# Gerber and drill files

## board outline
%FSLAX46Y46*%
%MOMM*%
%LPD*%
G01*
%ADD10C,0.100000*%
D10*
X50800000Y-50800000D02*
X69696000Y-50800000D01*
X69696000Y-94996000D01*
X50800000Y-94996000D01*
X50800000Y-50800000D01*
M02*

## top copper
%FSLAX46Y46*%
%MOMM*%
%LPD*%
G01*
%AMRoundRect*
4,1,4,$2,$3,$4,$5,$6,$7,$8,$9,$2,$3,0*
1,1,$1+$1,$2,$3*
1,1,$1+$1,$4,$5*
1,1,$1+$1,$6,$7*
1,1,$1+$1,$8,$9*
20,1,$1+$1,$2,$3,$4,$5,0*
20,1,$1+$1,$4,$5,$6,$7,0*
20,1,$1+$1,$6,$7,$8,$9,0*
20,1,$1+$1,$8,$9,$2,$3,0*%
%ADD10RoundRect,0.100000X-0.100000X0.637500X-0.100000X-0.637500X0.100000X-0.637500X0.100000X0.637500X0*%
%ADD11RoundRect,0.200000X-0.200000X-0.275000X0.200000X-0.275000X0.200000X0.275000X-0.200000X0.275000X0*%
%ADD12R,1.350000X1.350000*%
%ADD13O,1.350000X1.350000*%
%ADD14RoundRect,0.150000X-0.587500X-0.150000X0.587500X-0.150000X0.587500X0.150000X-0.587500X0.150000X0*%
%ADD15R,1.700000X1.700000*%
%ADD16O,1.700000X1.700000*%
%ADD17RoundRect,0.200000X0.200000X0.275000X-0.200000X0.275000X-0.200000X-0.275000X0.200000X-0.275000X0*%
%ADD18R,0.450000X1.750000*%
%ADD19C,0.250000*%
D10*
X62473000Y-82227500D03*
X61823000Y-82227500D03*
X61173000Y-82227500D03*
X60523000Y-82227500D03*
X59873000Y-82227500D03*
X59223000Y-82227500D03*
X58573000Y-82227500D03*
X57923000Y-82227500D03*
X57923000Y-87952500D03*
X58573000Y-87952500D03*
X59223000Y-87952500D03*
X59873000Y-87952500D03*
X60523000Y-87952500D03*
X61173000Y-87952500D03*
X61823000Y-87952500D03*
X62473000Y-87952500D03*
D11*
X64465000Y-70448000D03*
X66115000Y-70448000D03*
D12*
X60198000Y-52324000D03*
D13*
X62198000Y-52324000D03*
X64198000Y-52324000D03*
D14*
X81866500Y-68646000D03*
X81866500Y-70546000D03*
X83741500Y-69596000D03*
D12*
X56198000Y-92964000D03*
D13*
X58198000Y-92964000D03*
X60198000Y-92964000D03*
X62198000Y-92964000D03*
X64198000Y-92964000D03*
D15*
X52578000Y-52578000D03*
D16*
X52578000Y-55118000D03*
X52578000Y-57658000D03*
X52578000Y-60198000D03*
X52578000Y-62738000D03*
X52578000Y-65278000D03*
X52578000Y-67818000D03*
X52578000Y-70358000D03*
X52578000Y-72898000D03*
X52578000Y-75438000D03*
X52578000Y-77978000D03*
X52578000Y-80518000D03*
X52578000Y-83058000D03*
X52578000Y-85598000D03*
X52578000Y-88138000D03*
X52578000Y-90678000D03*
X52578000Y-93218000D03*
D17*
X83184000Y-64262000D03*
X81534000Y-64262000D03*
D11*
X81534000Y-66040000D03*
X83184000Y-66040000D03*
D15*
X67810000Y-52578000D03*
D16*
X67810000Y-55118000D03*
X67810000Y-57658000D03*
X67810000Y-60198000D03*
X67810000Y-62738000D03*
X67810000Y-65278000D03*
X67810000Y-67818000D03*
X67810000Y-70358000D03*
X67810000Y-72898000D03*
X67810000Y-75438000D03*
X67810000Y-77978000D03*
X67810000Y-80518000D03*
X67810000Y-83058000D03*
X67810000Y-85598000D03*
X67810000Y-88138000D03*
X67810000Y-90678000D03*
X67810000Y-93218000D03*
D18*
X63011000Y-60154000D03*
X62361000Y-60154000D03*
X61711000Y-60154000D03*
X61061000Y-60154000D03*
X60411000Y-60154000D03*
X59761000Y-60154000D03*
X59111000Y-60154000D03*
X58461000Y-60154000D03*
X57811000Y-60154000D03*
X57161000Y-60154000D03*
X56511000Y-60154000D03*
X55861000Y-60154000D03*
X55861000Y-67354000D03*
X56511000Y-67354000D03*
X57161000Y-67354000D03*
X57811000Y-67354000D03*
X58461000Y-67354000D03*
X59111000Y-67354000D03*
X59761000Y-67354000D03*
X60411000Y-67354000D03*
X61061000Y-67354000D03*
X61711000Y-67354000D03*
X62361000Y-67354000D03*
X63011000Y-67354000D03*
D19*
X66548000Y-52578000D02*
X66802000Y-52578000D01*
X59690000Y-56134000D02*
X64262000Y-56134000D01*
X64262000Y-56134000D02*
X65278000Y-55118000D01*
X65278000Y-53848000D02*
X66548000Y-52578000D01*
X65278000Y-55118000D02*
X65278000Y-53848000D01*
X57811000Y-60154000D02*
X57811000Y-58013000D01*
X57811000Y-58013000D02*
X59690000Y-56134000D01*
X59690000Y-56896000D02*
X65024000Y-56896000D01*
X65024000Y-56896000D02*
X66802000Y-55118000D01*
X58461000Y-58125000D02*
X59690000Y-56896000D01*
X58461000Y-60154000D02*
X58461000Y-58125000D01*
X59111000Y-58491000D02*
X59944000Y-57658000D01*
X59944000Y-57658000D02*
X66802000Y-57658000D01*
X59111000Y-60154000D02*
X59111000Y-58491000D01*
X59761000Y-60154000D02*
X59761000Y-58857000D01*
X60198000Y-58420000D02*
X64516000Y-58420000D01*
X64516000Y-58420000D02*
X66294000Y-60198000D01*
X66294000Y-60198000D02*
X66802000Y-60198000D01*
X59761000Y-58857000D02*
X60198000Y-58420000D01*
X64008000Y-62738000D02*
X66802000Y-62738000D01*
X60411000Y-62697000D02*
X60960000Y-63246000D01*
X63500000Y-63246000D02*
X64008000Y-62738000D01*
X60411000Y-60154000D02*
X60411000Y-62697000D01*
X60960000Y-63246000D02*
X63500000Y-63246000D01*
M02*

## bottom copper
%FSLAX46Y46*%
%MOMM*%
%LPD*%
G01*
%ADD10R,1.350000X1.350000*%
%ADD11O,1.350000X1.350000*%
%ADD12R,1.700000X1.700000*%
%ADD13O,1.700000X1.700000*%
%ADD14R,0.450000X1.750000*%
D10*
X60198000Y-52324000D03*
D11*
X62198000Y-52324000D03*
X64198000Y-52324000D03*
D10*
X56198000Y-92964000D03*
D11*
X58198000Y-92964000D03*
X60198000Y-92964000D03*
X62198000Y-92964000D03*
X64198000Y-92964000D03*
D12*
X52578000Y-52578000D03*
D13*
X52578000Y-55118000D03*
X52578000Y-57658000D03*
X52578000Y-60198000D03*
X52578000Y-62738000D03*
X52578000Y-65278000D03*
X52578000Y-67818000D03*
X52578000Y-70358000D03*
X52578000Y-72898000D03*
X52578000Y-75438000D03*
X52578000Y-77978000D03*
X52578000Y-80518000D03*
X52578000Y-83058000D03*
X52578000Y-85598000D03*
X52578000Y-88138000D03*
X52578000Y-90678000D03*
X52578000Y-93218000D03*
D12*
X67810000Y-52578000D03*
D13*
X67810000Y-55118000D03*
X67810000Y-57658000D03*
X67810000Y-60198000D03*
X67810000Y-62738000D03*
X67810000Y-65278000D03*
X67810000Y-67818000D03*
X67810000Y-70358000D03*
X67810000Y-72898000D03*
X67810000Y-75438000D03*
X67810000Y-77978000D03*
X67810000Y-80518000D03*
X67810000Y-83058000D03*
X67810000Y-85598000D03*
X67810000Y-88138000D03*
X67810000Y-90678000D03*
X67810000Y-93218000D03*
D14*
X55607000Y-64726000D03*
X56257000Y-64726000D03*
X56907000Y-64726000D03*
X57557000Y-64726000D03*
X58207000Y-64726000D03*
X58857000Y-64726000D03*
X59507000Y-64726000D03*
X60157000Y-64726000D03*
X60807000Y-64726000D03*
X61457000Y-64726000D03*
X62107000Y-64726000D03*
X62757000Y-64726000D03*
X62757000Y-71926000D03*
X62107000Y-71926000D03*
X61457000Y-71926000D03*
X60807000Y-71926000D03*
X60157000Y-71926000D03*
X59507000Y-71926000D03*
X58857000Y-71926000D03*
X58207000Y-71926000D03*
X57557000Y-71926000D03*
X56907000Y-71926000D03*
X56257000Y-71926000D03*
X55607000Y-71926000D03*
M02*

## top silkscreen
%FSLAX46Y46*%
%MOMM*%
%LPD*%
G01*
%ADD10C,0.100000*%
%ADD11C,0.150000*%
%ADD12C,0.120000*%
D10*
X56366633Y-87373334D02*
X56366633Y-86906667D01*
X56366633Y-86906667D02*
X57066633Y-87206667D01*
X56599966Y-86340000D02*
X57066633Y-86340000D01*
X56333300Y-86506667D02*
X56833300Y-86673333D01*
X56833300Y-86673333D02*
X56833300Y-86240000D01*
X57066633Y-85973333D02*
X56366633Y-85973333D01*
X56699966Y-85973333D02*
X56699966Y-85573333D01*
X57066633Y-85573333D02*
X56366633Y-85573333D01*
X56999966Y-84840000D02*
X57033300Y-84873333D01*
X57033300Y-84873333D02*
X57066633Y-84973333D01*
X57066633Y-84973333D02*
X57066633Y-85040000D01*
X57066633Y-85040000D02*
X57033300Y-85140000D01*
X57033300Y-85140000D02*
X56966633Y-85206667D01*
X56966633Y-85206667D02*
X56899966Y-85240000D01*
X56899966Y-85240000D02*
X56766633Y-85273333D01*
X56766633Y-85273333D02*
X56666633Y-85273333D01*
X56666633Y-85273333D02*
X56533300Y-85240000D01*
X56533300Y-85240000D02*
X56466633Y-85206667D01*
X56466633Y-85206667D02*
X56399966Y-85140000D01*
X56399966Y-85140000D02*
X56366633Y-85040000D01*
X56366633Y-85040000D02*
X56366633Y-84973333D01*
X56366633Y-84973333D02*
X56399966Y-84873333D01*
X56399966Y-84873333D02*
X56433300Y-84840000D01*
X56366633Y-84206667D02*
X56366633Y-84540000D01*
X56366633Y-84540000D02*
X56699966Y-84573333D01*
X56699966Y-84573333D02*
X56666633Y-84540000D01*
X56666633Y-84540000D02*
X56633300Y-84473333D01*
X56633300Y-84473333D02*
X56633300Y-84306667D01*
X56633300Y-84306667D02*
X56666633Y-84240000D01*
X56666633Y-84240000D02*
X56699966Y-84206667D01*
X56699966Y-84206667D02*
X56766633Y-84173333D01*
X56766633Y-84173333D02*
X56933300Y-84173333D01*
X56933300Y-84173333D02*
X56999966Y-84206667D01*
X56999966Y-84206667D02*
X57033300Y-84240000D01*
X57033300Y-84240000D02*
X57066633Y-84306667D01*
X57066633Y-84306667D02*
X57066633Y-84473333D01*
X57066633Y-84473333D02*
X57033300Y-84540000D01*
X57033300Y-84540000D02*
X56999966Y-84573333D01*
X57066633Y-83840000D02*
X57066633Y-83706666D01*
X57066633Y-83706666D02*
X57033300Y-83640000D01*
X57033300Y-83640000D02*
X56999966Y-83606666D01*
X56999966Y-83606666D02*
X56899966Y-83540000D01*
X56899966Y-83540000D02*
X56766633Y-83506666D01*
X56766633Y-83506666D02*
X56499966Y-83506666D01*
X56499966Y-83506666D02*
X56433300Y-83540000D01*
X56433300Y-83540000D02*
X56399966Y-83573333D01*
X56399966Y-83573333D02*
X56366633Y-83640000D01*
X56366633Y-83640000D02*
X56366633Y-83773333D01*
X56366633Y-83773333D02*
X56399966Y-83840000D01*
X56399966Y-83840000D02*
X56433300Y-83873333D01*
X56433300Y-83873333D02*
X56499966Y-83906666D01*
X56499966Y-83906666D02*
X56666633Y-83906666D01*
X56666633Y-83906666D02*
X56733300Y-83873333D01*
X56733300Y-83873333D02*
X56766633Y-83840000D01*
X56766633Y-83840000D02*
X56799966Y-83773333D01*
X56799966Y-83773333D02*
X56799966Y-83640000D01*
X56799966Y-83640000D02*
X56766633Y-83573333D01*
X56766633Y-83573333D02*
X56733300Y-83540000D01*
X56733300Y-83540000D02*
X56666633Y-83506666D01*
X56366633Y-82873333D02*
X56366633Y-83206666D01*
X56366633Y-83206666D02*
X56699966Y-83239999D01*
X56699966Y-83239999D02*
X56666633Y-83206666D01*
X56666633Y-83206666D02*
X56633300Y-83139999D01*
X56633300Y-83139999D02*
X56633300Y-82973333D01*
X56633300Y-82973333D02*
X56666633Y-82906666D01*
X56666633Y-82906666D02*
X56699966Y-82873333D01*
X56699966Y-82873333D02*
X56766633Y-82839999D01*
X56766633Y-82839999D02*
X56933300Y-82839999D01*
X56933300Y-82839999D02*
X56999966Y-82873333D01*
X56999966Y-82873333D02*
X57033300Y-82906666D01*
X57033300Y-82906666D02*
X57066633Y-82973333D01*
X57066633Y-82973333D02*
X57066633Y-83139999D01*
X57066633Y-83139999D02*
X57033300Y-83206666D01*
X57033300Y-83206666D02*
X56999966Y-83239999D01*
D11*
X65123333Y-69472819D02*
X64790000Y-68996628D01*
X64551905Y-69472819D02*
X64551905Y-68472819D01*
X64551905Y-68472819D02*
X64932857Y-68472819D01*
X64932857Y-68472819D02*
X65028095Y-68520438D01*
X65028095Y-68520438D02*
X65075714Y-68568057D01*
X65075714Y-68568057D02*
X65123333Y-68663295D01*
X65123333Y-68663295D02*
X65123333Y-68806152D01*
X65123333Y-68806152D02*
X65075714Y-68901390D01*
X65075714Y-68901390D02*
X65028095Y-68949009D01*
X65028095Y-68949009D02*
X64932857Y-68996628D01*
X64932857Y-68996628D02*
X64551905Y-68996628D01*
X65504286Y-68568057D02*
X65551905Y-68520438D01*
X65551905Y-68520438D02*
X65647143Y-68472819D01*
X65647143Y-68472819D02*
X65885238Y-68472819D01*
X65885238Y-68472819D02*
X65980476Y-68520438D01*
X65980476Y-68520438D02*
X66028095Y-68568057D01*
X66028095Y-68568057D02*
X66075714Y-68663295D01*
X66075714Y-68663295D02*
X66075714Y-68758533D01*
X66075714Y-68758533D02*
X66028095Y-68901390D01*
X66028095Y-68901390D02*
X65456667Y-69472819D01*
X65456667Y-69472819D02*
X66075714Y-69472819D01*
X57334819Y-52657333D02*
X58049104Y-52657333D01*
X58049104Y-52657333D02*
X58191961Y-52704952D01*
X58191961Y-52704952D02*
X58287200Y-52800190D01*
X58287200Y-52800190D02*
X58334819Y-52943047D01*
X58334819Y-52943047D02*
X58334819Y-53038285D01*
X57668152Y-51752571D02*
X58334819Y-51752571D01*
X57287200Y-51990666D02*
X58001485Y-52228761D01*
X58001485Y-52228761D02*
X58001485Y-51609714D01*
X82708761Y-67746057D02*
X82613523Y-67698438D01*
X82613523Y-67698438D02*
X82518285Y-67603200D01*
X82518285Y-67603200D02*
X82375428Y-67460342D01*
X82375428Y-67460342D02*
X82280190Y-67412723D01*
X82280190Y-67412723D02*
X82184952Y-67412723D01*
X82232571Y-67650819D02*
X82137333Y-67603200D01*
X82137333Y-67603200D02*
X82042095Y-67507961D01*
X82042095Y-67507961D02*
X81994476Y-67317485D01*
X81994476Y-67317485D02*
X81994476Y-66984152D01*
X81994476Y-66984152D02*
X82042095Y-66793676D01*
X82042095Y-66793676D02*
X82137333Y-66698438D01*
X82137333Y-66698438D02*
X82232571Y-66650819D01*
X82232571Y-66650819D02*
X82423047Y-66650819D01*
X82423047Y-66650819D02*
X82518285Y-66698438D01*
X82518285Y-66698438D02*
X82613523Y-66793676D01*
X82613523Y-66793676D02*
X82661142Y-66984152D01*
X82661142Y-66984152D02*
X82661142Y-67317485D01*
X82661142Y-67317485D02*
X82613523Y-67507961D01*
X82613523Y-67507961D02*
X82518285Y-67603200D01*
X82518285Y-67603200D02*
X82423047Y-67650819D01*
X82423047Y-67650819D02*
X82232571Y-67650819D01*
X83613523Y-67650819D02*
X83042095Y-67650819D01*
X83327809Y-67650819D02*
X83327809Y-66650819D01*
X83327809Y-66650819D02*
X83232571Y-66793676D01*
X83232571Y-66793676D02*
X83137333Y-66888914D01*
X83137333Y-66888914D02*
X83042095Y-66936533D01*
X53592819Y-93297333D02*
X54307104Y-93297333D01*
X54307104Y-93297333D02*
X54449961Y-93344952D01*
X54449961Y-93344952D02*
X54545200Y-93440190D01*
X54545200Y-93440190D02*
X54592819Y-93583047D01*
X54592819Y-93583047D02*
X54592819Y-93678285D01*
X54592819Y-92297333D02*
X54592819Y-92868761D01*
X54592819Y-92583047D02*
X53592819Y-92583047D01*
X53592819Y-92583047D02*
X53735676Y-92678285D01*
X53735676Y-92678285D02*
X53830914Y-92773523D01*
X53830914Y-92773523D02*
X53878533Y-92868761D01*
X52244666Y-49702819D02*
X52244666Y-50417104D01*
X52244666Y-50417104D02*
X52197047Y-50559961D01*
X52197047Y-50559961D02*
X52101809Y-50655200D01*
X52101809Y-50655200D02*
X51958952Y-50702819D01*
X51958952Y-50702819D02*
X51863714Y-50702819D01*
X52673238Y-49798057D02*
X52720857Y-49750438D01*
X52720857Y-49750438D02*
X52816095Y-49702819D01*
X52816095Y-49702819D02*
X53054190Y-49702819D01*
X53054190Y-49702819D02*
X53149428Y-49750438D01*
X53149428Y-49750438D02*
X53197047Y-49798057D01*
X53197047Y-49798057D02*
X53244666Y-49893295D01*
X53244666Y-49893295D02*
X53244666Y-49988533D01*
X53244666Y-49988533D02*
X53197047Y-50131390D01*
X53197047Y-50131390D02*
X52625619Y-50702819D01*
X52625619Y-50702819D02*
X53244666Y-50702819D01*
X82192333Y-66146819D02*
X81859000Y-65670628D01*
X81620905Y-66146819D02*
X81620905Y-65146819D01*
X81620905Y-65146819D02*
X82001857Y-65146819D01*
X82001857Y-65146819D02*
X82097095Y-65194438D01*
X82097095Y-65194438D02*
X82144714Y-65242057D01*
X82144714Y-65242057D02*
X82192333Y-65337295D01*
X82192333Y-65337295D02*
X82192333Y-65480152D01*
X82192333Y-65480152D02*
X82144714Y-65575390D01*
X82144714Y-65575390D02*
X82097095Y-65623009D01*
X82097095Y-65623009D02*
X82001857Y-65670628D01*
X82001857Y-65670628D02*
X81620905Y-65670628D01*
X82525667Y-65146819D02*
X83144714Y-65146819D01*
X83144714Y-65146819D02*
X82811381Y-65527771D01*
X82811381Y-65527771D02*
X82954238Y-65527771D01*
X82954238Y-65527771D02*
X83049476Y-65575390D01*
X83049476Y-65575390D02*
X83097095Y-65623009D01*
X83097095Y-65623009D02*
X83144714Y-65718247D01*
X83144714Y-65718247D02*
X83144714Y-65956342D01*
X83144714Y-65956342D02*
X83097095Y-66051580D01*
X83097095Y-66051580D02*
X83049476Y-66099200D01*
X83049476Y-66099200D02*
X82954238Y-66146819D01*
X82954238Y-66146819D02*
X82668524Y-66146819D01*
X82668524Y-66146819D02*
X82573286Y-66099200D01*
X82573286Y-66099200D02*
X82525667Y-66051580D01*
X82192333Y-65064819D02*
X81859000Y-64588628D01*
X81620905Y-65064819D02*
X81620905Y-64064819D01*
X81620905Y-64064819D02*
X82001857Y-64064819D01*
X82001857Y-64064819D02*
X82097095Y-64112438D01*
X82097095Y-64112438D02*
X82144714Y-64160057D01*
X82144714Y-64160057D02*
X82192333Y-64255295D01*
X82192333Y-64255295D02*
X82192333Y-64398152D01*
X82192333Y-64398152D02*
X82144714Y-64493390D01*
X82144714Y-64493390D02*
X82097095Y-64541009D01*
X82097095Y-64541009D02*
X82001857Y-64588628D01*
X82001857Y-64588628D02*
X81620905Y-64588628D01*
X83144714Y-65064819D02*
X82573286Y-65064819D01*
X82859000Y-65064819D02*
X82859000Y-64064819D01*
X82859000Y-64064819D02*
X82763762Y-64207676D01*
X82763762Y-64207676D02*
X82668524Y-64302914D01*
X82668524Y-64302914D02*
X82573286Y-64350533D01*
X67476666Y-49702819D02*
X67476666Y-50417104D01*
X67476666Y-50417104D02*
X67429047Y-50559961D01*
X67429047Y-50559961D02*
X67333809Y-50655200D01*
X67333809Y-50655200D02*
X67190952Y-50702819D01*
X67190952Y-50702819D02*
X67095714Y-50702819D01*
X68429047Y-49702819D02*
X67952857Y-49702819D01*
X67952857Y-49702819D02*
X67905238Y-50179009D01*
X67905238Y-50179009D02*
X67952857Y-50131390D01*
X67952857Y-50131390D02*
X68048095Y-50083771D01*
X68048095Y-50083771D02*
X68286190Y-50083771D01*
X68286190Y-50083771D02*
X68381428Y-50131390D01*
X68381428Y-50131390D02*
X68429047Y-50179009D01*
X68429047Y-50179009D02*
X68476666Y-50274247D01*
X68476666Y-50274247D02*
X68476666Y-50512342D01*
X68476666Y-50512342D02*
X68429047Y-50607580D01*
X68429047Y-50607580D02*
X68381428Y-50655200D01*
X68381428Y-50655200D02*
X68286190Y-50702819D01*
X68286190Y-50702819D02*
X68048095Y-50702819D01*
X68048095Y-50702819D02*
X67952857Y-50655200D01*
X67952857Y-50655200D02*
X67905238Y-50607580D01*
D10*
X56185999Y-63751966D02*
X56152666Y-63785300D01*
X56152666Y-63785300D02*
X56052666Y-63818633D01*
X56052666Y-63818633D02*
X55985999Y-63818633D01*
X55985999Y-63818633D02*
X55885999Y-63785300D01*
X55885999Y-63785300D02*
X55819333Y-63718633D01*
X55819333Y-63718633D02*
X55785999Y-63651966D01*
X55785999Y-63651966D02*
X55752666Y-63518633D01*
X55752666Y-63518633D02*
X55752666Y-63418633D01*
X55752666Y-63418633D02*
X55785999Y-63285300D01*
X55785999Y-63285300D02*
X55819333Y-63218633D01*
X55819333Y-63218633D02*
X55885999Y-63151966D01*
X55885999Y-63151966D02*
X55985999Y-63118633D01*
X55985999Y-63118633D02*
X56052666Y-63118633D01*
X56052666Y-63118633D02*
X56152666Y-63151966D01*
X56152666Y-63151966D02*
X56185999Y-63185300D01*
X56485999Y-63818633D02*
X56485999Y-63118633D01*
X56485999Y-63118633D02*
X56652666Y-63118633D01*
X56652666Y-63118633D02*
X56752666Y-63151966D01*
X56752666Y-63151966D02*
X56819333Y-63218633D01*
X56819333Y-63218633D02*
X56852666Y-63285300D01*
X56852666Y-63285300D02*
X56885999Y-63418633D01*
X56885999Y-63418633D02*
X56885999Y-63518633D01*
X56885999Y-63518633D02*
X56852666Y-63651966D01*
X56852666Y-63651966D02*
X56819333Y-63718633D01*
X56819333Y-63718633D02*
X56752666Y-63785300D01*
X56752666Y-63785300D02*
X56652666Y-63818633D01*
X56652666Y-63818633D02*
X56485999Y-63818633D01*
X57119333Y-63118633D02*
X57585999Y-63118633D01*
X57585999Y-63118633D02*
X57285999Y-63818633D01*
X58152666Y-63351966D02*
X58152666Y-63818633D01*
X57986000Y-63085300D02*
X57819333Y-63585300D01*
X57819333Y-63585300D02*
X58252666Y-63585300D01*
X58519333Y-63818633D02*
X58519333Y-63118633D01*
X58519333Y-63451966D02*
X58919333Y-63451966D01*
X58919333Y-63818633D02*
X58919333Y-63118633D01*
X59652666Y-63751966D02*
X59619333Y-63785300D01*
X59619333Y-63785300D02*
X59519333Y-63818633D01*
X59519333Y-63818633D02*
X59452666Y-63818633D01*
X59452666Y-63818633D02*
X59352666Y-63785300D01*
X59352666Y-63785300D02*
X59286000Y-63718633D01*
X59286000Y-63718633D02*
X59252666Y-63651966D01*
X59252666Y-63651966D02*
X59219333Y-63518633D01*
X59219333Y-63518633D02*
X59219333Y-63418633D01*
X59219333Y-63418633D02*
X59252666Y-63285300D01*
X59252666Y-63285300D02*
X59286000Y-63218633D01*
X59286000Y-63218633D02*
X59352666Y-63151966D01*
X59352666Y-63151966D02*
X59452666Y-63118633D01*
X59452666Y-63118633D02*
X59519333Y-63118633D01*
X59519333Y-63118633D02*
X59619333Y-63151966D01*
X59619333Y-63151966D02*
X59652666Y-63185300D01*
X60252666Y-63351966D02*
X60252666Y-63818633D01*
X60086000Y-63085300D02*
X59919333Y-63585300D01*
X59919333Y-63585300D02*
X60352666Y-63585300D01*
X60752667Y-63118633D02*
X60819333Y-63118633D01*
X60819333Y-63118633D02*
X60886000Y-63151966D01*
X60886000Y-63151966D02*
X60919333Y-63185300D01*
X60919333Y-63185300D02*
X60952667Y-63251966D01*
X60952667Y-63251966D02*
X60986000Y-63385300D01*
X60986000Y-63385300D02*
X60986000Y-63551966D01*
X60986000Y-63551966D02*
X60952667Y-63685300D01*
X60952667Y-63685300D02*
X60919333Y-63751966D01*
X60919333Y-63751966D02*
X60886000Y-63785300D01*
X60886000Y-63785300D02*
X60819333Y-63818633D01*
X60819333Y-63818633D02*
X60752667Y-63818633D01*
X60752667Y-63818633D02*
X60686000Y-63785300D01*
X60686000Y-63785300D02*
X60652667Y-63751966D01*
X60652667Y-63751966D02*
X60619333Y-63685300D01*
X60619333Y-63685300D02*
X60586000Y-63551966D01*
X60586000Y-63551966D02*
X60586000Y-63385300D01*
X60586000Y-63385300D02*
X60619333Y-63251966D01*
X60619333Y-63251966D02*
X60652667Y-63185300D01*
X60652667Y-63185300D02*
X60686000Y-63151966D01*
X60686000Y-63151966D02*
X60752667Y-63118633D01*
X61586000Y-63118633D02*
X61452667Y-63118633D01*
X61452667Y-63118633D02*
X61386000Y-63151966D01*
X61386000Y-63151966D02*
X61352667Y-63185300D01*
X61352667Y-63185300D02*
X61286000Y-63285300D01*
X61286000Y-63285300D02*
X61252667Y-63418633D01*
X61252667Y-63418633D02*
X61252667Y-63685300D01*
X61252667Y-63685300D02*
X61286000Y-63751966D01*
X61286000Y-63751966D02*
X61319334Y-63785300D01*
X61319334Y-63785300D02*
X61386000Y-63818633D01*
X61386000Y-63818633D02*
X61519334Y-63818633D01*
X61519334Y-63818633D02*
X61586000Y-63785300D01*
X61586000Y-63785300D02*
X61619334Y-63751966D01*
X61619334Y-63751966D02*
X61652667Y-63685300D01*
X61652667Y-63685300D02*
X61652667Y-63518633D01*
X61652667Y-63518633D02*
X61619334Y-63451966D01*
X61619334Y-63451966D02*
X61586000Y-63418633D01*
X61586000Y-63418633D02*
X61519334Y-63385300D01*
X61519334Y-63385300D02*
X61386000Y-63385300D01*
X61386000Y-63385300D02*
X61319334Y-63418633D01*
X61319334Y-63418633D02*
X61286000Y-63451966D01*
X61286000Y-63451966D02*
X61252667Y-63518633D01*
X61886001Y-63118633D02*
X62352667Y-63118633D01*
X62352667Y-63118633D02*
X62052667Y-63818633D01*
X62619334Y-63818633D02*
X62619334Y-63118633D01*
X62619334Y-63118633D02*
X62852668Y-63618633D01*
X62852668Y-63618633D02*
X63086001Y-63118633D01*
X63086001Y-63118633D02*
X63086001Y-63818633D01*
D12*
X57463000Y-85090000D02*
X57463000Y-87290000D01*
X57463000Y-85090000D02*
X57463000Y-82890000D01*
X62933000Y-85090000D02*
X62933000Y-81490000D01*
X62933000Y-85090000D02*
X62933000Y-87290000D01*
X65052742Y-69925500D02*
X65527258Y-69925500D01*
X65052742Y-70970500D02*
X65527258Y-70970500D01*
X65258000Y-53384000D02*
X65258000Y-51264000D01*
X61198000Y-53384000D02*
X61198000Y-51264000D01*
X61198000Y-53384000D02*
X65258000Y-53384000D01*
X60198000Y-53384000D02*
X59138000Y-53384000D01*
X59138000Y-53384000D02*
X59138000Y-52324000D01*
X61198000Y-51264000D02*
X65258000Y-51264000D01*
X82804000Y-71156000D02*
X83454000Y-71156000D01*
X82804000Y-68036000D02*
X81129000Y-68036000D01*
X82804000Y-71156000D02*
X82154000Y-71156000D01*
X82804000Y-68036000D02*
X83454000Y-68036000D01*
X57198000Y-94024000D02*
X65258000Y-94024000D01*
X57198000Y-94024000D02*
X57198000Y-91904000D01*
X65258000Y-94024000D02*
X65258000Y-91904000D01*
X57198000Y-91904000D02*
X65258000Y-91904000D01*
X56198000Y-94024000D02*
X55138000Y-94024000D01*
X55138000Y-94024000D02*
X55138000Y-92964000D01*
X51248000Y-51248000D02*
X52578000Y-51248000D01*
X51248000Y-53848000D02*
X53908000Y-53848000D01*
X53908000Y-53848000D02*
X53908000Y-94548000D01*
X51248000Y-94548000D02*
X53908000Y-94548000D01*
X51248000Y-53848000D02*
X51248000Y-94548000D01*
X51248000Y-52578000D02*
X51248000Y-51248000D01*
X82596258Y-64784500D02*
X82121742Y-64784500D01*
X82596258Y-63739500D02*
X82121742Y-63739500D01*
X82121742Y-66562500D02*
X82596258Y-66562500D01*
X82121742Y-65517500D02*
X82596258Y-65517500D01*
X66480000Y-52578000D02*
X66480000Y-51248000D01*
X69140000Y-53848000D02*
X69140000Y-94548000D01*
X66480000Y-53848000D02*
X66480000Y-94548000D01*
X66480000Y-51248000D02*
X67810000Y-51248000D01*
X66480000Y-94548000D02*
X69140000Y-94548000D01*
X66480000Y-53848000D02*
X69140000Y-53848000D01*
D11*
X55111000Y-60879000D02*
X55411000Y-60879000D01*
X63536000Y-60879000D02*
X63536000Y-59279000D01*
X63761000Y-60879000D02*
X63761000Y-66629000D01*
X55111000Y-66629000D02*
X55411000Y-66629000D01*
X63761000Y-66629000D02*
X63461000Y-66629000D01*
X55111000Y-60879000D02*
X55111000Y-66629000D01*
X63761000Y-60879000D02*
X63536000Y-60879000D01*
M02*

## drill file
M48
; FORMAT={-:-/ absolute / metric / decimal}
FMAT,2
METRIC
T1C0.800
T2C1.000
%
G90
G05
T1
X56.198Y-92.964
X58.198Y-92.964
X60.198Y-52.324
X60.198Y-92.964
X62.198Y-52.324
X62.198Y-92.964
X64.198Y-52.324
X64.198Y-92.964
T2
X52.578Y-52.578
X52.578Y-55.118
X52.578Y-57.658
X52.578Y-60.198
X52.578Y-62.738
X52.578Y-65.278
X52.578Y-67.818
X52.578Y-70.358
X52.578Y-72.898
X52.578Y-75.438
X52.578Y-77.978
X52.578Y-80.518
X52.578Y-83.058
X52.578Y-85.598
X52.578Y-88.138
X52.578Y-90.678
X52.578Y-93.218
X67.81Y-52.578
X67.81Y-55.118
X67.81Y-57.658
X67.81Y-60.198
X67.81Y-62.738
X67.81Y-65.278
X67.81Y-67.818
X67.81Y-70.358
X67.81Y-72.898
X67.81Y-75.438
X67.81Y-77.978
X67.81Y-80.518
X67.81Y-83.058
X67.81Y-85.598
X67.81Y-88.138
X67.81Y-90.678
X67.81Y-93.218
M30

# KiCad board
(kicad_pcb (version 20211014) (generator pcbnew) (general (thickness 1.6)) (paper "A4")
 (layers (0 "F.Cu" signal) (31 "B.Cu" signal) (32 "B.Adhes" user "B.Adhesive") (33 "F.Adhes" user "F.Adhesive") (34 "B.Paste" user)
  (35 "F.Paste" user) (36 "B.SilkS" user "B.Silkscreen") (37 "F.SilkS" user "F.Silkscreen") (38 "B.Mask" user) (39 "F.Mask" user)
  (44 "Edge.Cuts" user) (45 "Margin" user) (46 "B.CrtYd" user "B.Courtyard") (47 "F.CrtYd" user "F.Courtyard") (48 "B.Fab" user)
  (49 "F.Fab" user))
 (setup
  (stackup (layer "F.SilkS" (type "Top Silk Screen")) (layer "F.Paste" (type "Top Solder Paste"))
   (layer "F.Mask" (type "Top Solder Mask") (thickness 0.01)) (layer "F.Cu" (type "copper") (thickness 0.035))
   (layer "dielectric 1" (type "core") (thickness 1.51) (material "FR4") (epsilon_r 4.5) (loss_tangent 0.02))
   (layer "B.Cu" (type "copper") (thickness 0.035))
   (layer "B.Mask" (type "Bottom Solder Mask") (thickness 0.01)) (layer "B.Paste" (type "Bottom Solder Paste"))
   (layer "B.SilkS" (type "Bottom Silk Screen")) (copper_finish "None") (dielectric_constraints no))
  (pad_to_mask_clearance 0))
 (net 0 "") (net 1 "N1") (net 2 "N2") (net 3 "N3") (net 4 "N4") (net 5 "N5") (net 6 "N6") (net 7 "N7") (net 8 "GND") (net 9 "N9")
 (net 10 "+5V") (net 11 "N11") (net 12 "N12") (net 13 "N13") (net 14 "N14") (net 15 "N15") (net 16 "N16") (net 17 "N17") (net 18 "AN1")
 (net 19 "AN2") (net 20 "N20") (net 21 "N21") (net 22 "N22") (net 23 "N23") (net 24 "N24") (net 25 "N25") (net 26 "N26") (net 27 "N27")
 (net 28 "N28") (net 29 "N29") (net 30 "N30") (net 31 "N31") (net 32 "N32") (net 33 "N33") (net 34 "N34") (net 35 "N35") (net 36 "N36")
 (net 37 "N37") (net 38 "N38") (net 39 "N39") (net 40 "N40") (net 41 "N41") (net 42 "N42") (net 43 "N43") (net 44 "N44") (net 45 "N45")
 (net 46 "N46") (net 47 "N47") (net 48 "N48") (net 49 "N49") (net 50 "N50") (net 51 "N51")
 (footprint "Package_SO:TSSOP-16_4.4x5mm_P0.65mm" (layer "F.Cu") (at 60.198 85.09 -90)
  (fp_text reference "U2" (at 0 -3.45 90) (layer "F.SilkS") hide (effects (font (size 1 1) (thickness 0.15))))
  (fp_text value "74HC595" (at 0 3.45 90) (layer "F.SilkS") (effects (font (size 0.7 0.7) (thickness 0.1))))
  (fp_line (start 0 2.735) (end 2.2 2.735) (layer "F.SilkS") (width 0.12))
  (fp_line (start 0 2.735) (end -2.2 2.735) (layer "F.SilkS") (width 0.12))
  (fp_line (start 0 -2.735) (end -3.6 -2.735) (layer "F.SilkS") (width 0.12))
  (fp_line (start 0 -2.735) (end 2.2 -2.735) (layer "F.SilkS") (width 0.12))
  (pad "1" smd roundrect (at -2.8625 -2.275 270) (size 1.475 0.4) (layers "F.Cu" "F.Paste" "F.Mask") (roundrect_rratio 0.25) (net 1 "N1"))
  (pad "2" smd roundrect (at -2.8625 -1.625 270) (size 1.475 0.4) (layers "F.Cu" "F.Paste" "F.Mask") (roundrect_rratio 0.25) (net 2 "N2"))
  (pad "3" smd roundrect (at -2.8625 -0.975 270) (size 1.475 0.4) (layers "F.Cu" "F.Paste" "F.Mask") (roundrect_rratio 0.25) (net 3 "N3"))
  (pad "4" smd roundrect (at -2.8625 -0.325 270) (size 1.475 0.4) (layers "F.Cu" "F.Paste" "F.Mask") (roundrect_rratio 0.25) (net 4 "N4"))
  (pad "5" smd roundrect (at -2.8625 0.325 270) (size 1.475 0.4) (layers "F.Cu" "F.Paste" "F.Mask") (roundrect_rratio 0.25) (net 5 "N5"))
  (pad "6" smd roundrect (at -2.8625 0.975 270) (size 1.475 0.4) (layers "F.Cu" "F.Paste" "F.Mask") (roundrect_rratio 0.25) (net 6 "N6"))
  (pad "7" smd roundrect (at -2.8625 1.625 270) (size 1.475 0.4) (layers "F.Cu" "F.Paste" "F.Mask") (roundrect_rratio 0.25) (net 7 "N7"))
  (pad "8" smd roundrect (at -2.8625 2.275 270) (size 1.475 0.4) (layers "F.Cu" "F.Paste" "F.Mask") (roundrect_rratio 0.25) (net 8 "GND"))
  (pad "9" smd roundrect (at 2.8625 2.275 270) (size 1.475 0.4) (layers "F.Cu" "F.Paste" "F.Mask") (roundrect_rratio 0.25) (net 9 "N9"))
  (pad "10" smd roundrect (at 2.8625 1.625 270) (size 1.475 0.4) (layers "F.Cu" "F.Paste" "F.Mask") (roundrect_rratio 0.25) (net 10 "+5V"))
  (pad "11" smd roundrect (at 2.8625 0.975 270) (size 1.475 0.4) (layers "F.Cu" "F.Paste" "F.Mask") (roundrect_rratio 0.25) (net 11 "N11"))
  (pad "12" smd roundrect (at 2.8625 0.325 270) (size 1.475 0.4) (layers "F.Cu" "F.Paste" "F.Mask") (roundrect_rratio 0.25) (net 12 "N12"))
  (pad "13" smd roundrect (at 2.8625 -0.325 270) (size 1.475 0.4) (layers "F.Cu" "F.Paste" "F.Mask") (roundrect_rratio 0.25) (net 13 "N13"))
  (pad "14" smd roundrect (at 2.8625 -0.975 270) (size 1.475 0.4) (layers "F.Cu" "F.Paste" "F.Mask") (roundrect_rratio 0.25) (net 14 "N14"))
  (pad "15" smd roundrect (at 2.8625 -1.625 270) (size 1.475 0.4) (layers "F.Cu" "F.Paste" "F.Mask") (roundrect_rratio 0.25) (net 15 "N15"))
  (pad "16" smd roundrect (at 2.8625 -2.275 270) (size 1.475 0.4) (layers "F.Cu" "F.Paste" "F.Mask") (roundrect_rratio 0.25) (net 10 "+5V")))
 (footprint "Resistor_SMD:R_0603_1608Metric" (layer "F.Cu") (at 65.29 70.448)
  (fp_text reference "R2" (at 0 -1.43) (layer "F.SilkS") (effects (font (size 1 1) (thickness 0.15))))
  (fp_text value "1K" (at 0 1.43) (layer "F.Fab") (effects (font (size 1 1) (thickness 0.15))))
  (fp_line (start -0.237258 -0.5225) (end 0.237258 -0.5225) (layer "F.SilkS") (width 0.12))
  (fp_line (start -0.237258 0.5225) (end 0.237258 0.5225) (layer "F.SilkS") (width 0.12))
  (pad "1" smd roundrect (at -0.825 0) (size 0.8 0.95) (layers "F.Cu" "F.Paste" "F.Mask") (roundrect_rratio 0.25) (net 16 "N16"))
  (pad "2" smd roundrect (at 0.825 0) (size 0.8 0.95) (layers "F.Cu" "F.Paste" "F.Mask") (roundrect_rratio 0.25) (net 13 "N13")))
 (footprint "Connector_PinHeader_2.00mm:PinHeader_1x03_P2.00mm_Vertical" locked (layer "F.Cu") (at 60.198 52.324 90)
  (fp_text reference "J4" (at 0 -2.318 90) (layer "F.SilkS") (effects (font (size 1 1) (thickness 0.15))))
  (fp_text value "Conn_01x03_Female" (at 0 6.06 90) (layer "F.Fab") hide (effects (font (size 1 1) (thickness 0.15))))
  (fp_line (start -1.06 5.06) (end 1.06 5.06) (layer "F.SilkS") (width 0.12))
  (fp_line (start -1.06 1) (end 1.06 1) (layer "F.SilkS") (width 0.12))
  (fp_line (start -1.06 1) (end -1.06 5.06) (layer "F.SilkS") (width 0.12))
  (fp_line (start -1.06 0) (end -1.06 -1.06) (layer "F.SilkS") (width 0.12))
  (fp_line (start -1.06 -1.06) (end 0 -1.06) (layer "F.SilkS") (width 0.12))
  (fp_line (start 1.06 1) (end 1.06 5.06) (layer "F.SilkS") (width 0.12))
  (pad "1" thru_hole rect locked (at 0 0 90) (size 1.35 1.35) (drill 0.8) (layers *.Cu *.Mask) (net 9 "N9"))
  (pad "2" thru_hole oval locked (at 0 2 90) (size 1.35 1.35) (drill 0.8) (layers *.Cu *.Mask) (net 12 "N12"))
  (pad "3" thru_hole oval locked (at 0 4 90) (size 1.35 1.35) (drill 0.8) (layers *.Cu *.Mask) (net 13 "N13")))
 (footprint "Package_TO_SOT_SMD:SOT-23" (layer "F.Cu") (at 82.804 69.596)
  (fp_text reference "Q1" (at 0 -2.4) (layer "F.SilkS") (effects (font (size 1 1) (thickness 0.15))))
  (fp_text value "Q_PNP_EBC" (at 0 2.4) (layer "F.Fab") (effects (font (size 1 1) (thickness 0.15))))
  (fp_line (start 0 1.56) (end 0.65 1.56) (layer "F.SilkS") (width 0.12))
  (fp_line (start 0 -1.56) (end -1.675 -1.56) (layer "F.SilkS") (width 0.12))
  (fp_line (start 0 1.56) (end -0.65 1.56) (layer "F.SilkS") (width 0.12))
  (fp_line (start 0 -1.56) (end 0.65 -1.56) (layer "F.SilkS") (width 0.12))
  (pad "1" smd roundrect (at -0.9375 -0.95) (size 1.475 0.6) (layers "F.Cu" "F.Paste" "F.Mask") (roundrect_rratio 0.25) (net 10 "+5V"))
  (pad "2" smd roundrect (at -0.9375 0.95) (size 1.475 0.6) (layers "F.Cu" "F.Paste" "F.Mask") (roundrect_rratio 0.25) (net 16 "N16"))
  (pad "3" smd roundrect (at 0.9375 0) (size 1.475 0.6) (layers "F.Cu" "F.Paste" "F.Mask") (roundrect_rratio 0.25) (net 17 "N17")))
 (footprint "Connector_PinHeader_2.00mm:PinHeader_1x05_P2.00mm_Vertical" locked (layer "F.Cu") (at 56.198 92.964 90)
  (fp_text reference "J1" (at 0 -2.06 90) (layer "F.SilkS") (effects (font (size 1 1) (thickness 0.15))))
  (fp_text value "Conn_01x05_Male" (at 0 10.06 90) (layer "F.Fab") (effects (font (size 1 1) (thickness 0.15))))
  (fp_line (start -1.06 1) (end -1.06 9.06) (layer "F.SilkS") (width 0.12))
  (fp_line (start -1.06 1) (end 1.06 1) (layer "F.SilkS") (width 0.12))
  (fp_line (start -1.06 9.06) (end 1.06 9.06) (layer "F.SilkS") (width 0.12))
  (fp_line (start 1.06 1) (end 1.06 9.06) (layer "F.SilkS") (width 0.12))
  (fp_line (start -1.06 0) (end -1.06 -1.06) (layer "F.SilkS") (width 0.12))
  (fp_line (start -1.06 -1.06) (end 0 -1.06) (layer "F.SilkS") (width 0.12))
  (pad "1" thru_hole rect locked (at 0 0 90) (size 1.35 1.35) (drill 0.8) (layers *.Cu *.Mask) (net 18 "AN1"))
  (pad "2" thru_hole oval locked (at 0 2 90) (size 1.35 1.35) (drill 0.8) (layers *.Cu *.Mask) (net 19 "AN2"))
  (pad "3" thru_hole oval locked (at 0 4 90) (size 1.35 1.35) (drill 0.8) (layers *.Cu *.Mask) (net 14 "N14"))
  (pad "4" thru_hole oval locked (at 0 6 90) (size 1.35 1.35) (drill 0.8) (layers *.Cu *.Mask) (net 11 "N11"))
  (pad "5" thru_hole oval locked (at 0 8 90) (size 1.35 1.35) (drill 0.8) (layers *.Cu *.Mask) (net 13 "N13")))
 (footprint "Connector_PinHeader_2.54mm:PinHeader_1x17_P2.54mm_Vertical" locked (layer "F.Cu") (at 52.578 52.578)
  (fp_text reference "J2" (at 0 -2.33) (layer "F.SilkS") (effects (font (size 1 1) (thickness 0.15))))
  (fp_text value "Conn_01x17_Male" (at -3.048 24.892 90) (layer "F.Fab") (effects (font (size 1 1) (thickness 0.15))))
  (fp_line (start -1.33 -1.33) (end 0 -1.33) (layer "F.SilkS") (width 0.12))
  (fp_line (start -1.33 1.27) (end 1.33 1.27) (layer "F.SilkS") (width 0.12))
  (fp_line (start 1.33 1.27) (end 1.33 41.97) (layer "F.SilkS") (width 0.12))
  (fp_line (start -1.33 41.97) (end 1.33 41.97) (layer "F.SilkS") (width 0.12))
  (fp_line (start -1.33 1.27) (end -1.33 41.97) (layer "F.SilkS") (width 0.12))
  (fp_line (start -1.33 0) (end -1.33 -1.33) (layer "F.SilkS") (width 0.12))
  (pad "1" thru_hole rect locked (at 0 0) (size 1.7 1.7) (drill 1) (layers *.Cu *.Mask) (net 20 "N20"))
  (pad "2" thru_hole oval locked (at 0 2.54) (size 1.7 1.7) (drill 1) (layers *.Cu *.Mask) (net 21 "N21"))
  (pad "3" thru_hole oval locked (at 0 5.08) (size 1.7 1.7) (drill 1) (layers *.Cu *.Mask) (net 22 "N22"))
  (pad "4" thru_hole oval locked (at 0 7.62) (size 1.7 1.7) (drill 1) (layers *.Cu *.Mask) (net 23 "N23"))
  (pad "5" thru_hole oval locked (at 0 10.16) (size 1.7 1.7) (drill 1) (layers *.Cu *.Mask) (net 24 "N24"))
  (pad "6" thru_hole oval locked (at 0 12.7) (size 1.7 1.7) (drill 1) (layers *.Cu *.Mask) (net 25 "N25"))
  (pad "7" thru_hole oval locked (at 0 15.24) (size 1.7 1.7) (drill 1) (layers *.Cu *.Mask) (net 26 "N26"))
  (pad "8" thru_hole oval locked (at 0 17.78) (size 1.7 1.7) (drill 1) (layers *.Cu *.Mask) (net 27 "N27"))
  (pad "9" thru_hole oval locked (at 0 20.32) (size 1.7 1.7) (drill 1) (layers *.Cu *.Mask) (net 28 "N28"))
  (pad "10" thru_hole oval locked (at 0 22.86) (size 1.7 1.7) (drill 1) (layers *.Cu *.Mask) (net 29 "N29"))
  (pad "11" thru_hole oval locked (at 0 25.4) (size 1.7 1.7) (drill 1) (layers *.Cu *.Mask) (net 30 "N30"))
  (pad "12" thru_hole oval locked (at 0 27.94) (size 1.7 1.7) (drill 1) (layers *.Cu *.Mask) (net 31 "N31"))
  (pad "13" thru_hole oval locked (at 0 30.48) (size 1.7 1.7) (drill 1) (layers *.Cu *.Mask) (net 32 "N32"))
  (pad "14" thru_hole oval locked (at 0 33.02) (size 1.7 1.7) (drill 1) (layers *.Cu *.Mask) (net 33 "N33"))
  (pad "15" thru_hole oval locked (at 0 35.56) (size 1.7 1.7) (drill 1) (layers *.Cu *.Mask) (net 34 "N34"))
  (pad "16" thru_hole oval locked (at 0 38.1) (size 1.7 1.7) (drill 1) (layers *.Cu *.Mask) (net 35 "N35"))
  (pad "17" thru_hole oval locked (at 0 40.64) (size 1.7 1.7) (drill 1) (layers *.Cu *.Mask) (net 8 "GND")))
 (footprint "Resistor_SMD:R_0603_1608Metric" (layer "F.Cu") (at 82.359 64.262 180)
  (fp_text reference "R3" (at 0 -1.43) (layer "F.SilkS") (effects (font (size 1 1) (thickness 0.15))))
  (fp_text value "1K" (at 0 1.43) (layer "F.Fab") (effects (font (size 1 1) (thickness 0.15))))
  (fp_line (start -0.237258 -0.5225) (end 0.237258 -0.5225) (layer "F.SilkS") (width 0.12))
  (fp_line (start -0.237258 0.5225) (end 0.237258 0.5225) (layer "F.SilkS") (width 0.12))
  (pad "1" smd roundrect (at -0.825 0 180) (size 0.8 0.95) (layers "F.Cu" "F.Paste" "F.Mask") (roundrect_rratio 0.25) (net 8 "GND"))
  (pad "2" smd roundrect (at 0.825 0 180) (size 0.8 0.95) (layers "F.Cu" "F.Paste" "F.Mask") (roundrect_rratio 0.25) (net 17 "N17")))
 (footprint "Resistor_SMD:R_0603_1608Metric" (layer "F.Cu") (at 82.359 66.04)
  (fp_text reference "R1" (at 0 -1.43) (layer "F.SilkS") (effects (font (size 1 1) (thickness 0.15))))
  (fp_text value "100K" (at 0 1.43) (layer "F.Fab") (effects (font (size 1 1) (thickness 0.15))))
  (fp_line (start -0.237258 0.5225) (end 0.237258 0.5225) (layer "F.SilkS") (width 0.12))
  (fp_line (start -0.237258 -0.5225) (end 0.237258 -0.5225) (layer "F.SilkS") (width 0.12))
  (pad "1" smd roundrect (at -0.825 0) (size 0.8 0.95) (layers "F.Cu" "F.Paste" "F.Mask") (roundrect_rratio 0.25) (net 10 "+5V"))
  (pad "2" smd roundrect (at 0.825 0) (size 0.8 0.95) (layers "F.Cu" "F.Paste" "F.Mask") (roundrect_rratio 0.25) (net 13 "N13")))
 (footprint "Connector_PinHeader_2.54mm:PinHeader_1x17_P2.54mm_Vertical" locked (layer "F.Cu") (at 67.81 52.578)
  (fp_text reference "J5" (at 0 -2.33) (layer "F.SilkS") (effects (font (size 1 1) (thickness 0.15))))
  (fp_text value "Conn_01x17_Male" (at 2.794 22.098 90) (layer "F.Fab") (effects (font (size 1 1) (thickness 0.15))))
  (fp_line (start -1.33 0) (end -1.33 -1.33) (layer "F.SilkS") (width 0.12))
  (fp_line (start 1.33 1.27) (end 1.33 41.97) (layer "F.SilkS") (width 0.12))
  (fp_line (start -1.33 1.27) (end -1.33 41.97) (layer "F.SilkS") (width 0.12))
  (fp_line (start -1.33 -1.33) (end 0 -1.33) (layer "F.SilkS") (width 0.12))
  (fp_line (start -1.33 41.97) (end 1.33 41.97) (layer "F.SilkS") (width 0.12))
  (fp_line (start -1.33 1.27) (end 1.33 1.27) (layer "F.SilkS") (width 0.12))
  (pad "1" thru_hole rect locked (at 0 0) (size 1.7 1.7) (drill 1) (layers *.Cu *.Mask) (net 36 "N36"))
  (pad "2" thru_hole oval locked (at 0 2.54) (size 1.7 1.7) (drill 1) (layers *.Cu *.Mask) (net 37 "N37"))
  (pad "3" thru_hole oval locked (at 0 5.08) (size 1.7 1.7) (drill 1) (layers *.Cu *.Mask) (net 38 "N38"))
  (pad "4" thru_hole oval locked (at 0 7.62) (size 1.7 1.7) (drill 1) (layers *.Cu *.Mask) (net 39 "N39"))
  (pad "5" thru_hole oval locked (at 0 10.16) (size 1.7 1.7) (drill 1) (layers *.Cu *.Mask) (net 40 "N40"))
  (pad "6" thru_hole oval locked (at 0 12.7) (size 1.7 1.7) (drill 1) (layers *.Cu *.Mask) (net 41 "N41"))
  (pad "7" thru_hole oval locked (at 0 15.24) (size 1.7 1.7) (drill 1) (layers *.Cu *.Mask) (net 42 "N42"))
  (pad "8" thru_hole oval locked (at 0 17.78) (size 1.7 1.7) (drill 1) (layers *.Cu *.Mask) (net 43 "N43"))
  (pad "9" thru_hole oval locked (at 0 20.32) (size 1.7 1.7) (drill 1) (layers *.Cu *.Mask) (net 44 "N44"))
  (pad "10" thru_hole oval locked (at 0 22.86) (size 1.7 1.7) (drill 1) (layers *.Cu *.Mask) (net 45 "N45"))
  (pad "11" thru_hole oval locked (at 0 25.4) (size 1.7 1.7) (drill 1) (layers *.Cu *.Mask) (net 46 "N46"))
  (pad "12" thru_hole oval locked (at 0 27.94) (size 1.7 1.7) (drill 1) (layers *.Cu *.Mask) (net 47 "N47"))
  (pad "13" thru_hole oval locked (at 0 30.48) (size 1.7 1.7) (drill 1) (layers *.Cu *.Mask) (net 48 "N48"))
  (pad "14" thru_hole oval locked (at 0 33.02) (size 1.7 1.7) (drill 1) (layers *.Cu *.Mask) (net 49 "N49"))
  (pad "15" thru_hole oval locked (at 0 35.56) (size 1.7 1.7) (drill 1) (layers *.Cu *.Mask) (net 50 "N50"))
  (pad "16" thru_hole oval locked (at 0 38.1) (size 1.7 1.7) (drill 1) (layers *.Cu *.Mask) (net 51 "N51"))
  (pad "17" thru_hole oval locked (at 0 40.64) (size 1.7 1.7) (drill 1) (layers *.Cu *.Mask) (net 10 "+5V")))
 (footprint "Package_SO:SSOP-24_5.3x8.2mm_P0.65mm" (layer "F.Cu") (at 59.436 63.754 -90)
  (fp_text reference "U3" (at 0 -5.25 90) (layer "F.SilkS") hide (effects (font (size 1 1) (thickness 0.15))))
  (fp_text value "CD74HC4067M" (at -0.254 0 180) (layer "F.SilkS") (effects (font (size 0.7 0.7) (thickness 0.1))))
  (fp_line (start -2.875 4.325) (end -2.875 4.025) (layer "F.SilkS") (width 0.15))
  (fp_line (start -2.875 -4.1) (end -4.475 -4.1) (layer "F.SilkS") (width 0.15))
  (fp_line (start -2.875 -4.325) (end 2.875 -4.325) (layer "F.SilkS") (width 0.15))
  (fp_line (start 2.875 4.325) (end 2.875 4.025) (layer "F.SilkS") (width 0.15))
  (fp_line (start 2.875 -4.325) (end 2.875 -4.025) (layer "F.SilkS") (width 0.15))
  (fp_line (start -2.875 4.325) (end 2.875 4.325) (layer "F.SilkS") (width 0.15))
  (fp_line (start -2.875 -4.325) (end -2.875 -4.1) (layer "F.SilkS") (width 0.15))
  (pad "1" smd rect (at -3.6 -3.575 270) (size 1.75 0.45) (layers "F.Cu" "F.Paste" "F.Mask") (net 19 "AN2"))
  (pad "2" smd rect (at -3.6 -2.925 270) (size 1.75 0.45) (layers "F.Cu" "F.Paste" "F.Mask") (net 43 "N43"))
  (pad "3" smd rect (at -3.6 -2.275 270) (size 1.75 0.45) (layers "F.Cu" "F.Paste" "F.Mask") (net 42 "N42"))
  (pad "4" smd rect (at -3.6 -1.625 270) (size 1.75 0.45) (layers "F.Cu" "F.Paste" "F.Mask") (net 41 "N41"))
  (pad "5" smd rect (at -3.6 -0.975 270) (size 1.75 0.45) (layers "F.Cu" "F.Paste" "F.Mask") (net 40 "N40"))
  (pad "6" smd rect (at -3.6 -0.325 270) (size 1.75 0.45) (layers "F.Cu" "F.Paste" "F.Mask") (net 39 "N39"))
  (pad "7" smd rect (at -3.6 0.325 270) (size 1.75 0.45) (layers "F.Cu" "F.Paste" "F.Mask") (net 38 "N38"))
  (pad "8" smd rect (at -3.6 0.975 270) (size 1.75 0.45) (layers "F.Cu" "F.Paste" "F.Mask") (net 37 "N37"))
  (pad "9" smd rect (at -3.6 1.625 270) (size 1.75 0.45) (layers "F.Cu" "F.Paste" "F.Mask") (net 36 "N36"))
  (pad "10" smd rect (at -3.6 2.275 270) (size 1.75 0.45) (layers "F.Cu" "F.Paste" "F.Mask") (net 4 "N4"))
  (pad "11" smd rect (at -3.6 2.925 270) (size 1.75 0.45) (layers "F.Cu" "F.Paste" "F.Mask") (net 5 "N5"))
  (pad "12" smd rect (at -3.6 3.575 270) (size 1.75 0.45) (layers "F.Cu" "F.Paste" "F.Mask") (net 8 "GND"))
  (pad "13" smd rect (at 3.6 3.575 270) (size 1.75 0.45) (layers "F.Cu" "F.Paste" "F.Mask") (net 7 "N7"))
  (pad "14" smd rect (at 3.6 2.925 270) (size 1.75 0.45) (layers "F.Cu" "F.Paste" "F.Mask") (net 6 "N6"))
  (pad "15" smd rect (at 3.6 2.275 270) (size 1.75 0.45) (layers "F.Cu" "F.Paste" "F.Mask") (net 17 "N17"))
  (pad "16" smd rect (at 3.6 1.625 270) (size 1.75 0.45) (layers "F.Cu" "F.Paste" "F.Mask") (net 51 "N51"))
  (pad "17" smd rect (at 3.6 0.975 270) (size 1.75 0.45) (layers "F.Cu" "F.Paste" "F.Mask") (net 50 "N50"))
  (pad "18" smd rect (at 3.6 0.325 270) (size 1.75 0.45) (layers "F.Cu" "F.Paste" "F.Mask") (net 49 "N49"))
  (pad "19" smd rect (at 3.6 -0.325 270) (size 1.75 0.45) (layers "F.Cu" "F.Paste" "F.Mask") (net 48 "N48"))
  (pad "20" smd rect (at 3.6 -0.975 270) (size 1.75 0.45) (layers "F.Cu" "F.Paste" "F.Mask") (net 47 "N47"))
  (pad "21" smd rect (at 3.6 -1.625 270) (size 1.75 0.45) (layers "F.Cu" "F.Paste" "F.Mask") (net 46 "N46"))
  (pad "22" smd rect (at 3.6 -2.275 270) (size 1.75 0.45) (layers "F.Cu" "F.Paste" "F.Mask") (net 45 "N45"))
  (pad "23" smd rect (at 3.6 -2.925 270) (size 1.75 0.45) (layers "F.Cu" "F.Paste" "F.Mask") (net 44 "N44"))
  (pad "24" smd rect (at 3.6 -3.575 270) (size 1.75 0.45) (layers "F.Cu" "F.Paste" "F.Mask") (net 10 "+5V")))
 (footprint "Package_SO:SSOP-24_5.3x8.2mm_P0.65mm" (layer "B.Cu") (at 59.182 68.326 -90)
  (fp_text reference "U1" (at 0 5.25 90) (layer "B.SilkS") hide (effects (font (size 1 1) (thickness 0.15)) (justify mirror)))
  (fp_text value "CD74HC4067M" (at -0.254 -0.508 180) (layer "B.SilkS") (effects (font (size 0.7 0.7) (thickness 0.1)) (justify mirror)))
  (pad "1" smd rect (at -3.6 3.575 270) (size 1.75 0.45) (layers "B.Cu" "B.Paste" "B.Mask") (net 18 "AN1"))
  (pad "2" smd rect (at -3.6 2.925 270) (size 1.75 0.45) (layers "B.Cu" "B.Paste" "B.Mask") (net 27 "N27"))
  (pad "3" smd rect (at -3.6 2.275 270) (size 1.75 0.45) (layers "B.Cu" "B.Paste" "B.Mask") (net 26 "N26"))
  (pad "4" smd rect (at -3.6 1.625 270) (size 1.75 0.45) (layers "B.Cu" "B.Paste" "B.Mask") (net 25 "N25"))
  (pad "5" smd rect (at -3.6 0.975 270) (size 1.75 0.45) (layers "B.Cu" "B.Paste" "B.Mask") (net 24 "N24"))
  (pad "6" smd rect (at -3.6 0.325 270) (size 1.75 0.45) (layers "B.Cu" "B.Paste" "B.Mask") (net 23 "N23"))
  (pad "7" smd rect (at -3.6 -0.325 270) (size 1.75 0.45) (layers "B.Cu" "B.Paste" "B.Mask") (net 22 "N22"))
  (pad "8" smd rect (at -3.6 -0.975 270) (size 1.75 0.45) (layers "B.Cu" "B.Paste" "B.Mask") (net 21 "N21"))
  (pad "9" smd rect (at -3.6 -1.625 270) (size 1.75 0.45) (layers "B.Cu" "B.Paste" "B.Mask") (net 20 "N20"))
  (pad "10" smd rect (at -3.6 -2.275 270) (size 1.75 0.45) (layers "B.Cu" "B.Paste" "B.Mask") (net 15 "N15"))
  (pad "11" smd rect (at -3.6 -2.925 270) (size 1.75 0.45) (layers "B.Cu" "B.Paste" "B.Mask") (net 1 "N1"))
  (pad "12" smd rect (at -3.6 -3.575 270) (size 1.75 0.45) (layers "B.Cu" "B.Paste" "B.Mask") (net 8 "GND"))
  (pad "13" smd rect (at 3.6 -3.575 270) (size 1.75 0.45) (layers "B.Cu" "B.Paste" "B.Mask") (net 3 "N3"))
  (pad "14" smd rect (at 3.6 -2.925 270) (size 1.75 0.45) (layers "B.Cu" "B.Paste" "B.Mask") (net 2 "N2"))
  (pad "15" smd rect (at 3.6 -2.275 270) (size 1.75 0.45) (layers "B.Cu" "B.Paste" "B.Mask") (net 17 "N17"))
  (pad "16" smd rect (at 3.6 -1.625 270) (size 1.75 0.45) (layers "B.Cu" "B.Paste" "B.Mask") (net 35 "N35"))
  (pad "17" smd rect (at 3.6 -0.975 270) (size 1.75 0.45) (layers "B.Cu" "B.Paste" "B.Mask") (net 34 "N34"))
  (pad "18" smd rect (at 3.6 -0.325 270) (size 1.75 0.45) (layers "B.Cu" "B.Paste" "B.Mask") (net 33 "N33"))
  (pad "19" smd rect (at 3.6 0.325 270) (size 1.75 0.45) (layers "B.Cu" "B.Paste" "B.Mask") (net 32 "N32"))
  (pad "20" smd rect (at 3.6 0.975 270) (size 1.75 0.45) (layers "B.Cu" "B.Paste" "B.Mask") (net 31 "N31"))
  (pad "21" smd rect (at 3.6 1.625 270) (size 1.75 0.45) (layers "B.Cu" "B.Paste" "B.Mask") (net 30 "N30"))
  (pad "22" smd rect (at 3.6 2.275 270) (size 1.75 0.45) (layers "B.Cu" "B.Paste" "B.Mask") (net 29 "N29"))
  (pad "23" smd rect (at 3.6 2.925 270) (size 1.75 0.45) (layers "B.Cu" "B.Paste" "B.Mask") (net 28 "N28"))
  (pad "24" smd rect (at 3.6 3.575 270) (size 1.75 0.45) (layers "B.Cu" "B.Paste" "B.Mask") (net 10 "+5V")))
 (gr_rect locked (start 50.8 50.8) (end 69.696 94.996) (layer "Edge.Cuts") (width 0.1) (fill none))
 (segment (start 66.548 52.578) (end 66.802 52.578) (width 0.25) (layer "F.Cu") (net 36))
 (segment (start 59.69 56.134) (end 64.262 56.134) (width 0.25) (layer "F.Cu") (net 36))
 (segment (start 64.262 56.134) (end 65.278 55.118) (width 0.25) (layer "F.Cu") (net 36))
 (segment (start 65.278 53.848) (end 66.548 52.578) (width 0.25) (layer "F.Cu") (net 36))
 (segment (start 65.278 55.118) (end 65.278 53.848) (width 0.25) (layer "F.Cu") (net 36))
 (segment (start 57.811 60.154) (end 57.811 58.013) (width 0.25) (layer "F.Cu") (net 36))
 (segment (start 57.811 58.013) (end 59.69 56.134) (width 0.25) (layer "F.Cu") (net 36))
 (segment (start 59.69 56.896) (end 65.024 56.896) (width 0.25) (layer "F.Cu") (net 37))
 (segment (start 65.024 56.896) (end 66.802 55.118) (width 0.25) (layer "F.Cu") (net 37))
 (segment (start 58.461 58.125) (end 59.69 56.896) (width 0.25) (layer "F.Cu") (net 37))
 (segment (start 58.461 60.154) (end 58.461 58.125) (width 0.25) (layer "F.Cu") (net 37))
 (segment (start 59.111 58.491) (end 59.944 57.658) (width 0.25) (layer "F.Cu") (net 38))
 (segment (start 59.944 57.658) (end 66.802 57.658) (width 0.25) (layer "F.Cu") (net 38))
 (segment (start 59.111 60.154) (end 59.111 58.491) (width 0.25) (layer "F.Cu") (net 38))
 (segment (start 59.761 60.154) (end 59.761 58.857) (width 0.25) (layer "F.Cu") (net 39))
 (segment (start 60.198 58.42) (end 64.516 58.42) (width 0.25) (layer "F.Cu") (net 39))
 (segment (start 64.516 58.42) (end 66.294 60.198) (width 0.25) (layer "F.Cu") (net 39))
 (segment (start 66.294 60.198) (end 66.802 60.198) (width 0.25) (layer "F.Cu") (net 39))
 (segment (start 59.761 58.857) (end 60.198 58.42) (width 0.25) (layer "F.Cu") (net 39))
 (segment (start 64.008 62.738) (end 66.802 62.738) (width 0.25) (layer "F.Cu") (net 40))
 (segment (start 60.411 62.697) (end 60.96 63.246) (width 0.25) (layer "F.Cu") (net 40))
 (segment (start 63.5 63.246) (end 64.008 62.738) (width 0.25) (layer "F.Cu") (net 40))
 (segment (start 60.411 60.154) (end 60.411 62.697) (width 0.25) (layer "F.Cu") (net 40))
 (segment (start 60.96 63.246) (end 63.5 63.246) (width 0.25) (layer "F.Cu") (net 40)))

